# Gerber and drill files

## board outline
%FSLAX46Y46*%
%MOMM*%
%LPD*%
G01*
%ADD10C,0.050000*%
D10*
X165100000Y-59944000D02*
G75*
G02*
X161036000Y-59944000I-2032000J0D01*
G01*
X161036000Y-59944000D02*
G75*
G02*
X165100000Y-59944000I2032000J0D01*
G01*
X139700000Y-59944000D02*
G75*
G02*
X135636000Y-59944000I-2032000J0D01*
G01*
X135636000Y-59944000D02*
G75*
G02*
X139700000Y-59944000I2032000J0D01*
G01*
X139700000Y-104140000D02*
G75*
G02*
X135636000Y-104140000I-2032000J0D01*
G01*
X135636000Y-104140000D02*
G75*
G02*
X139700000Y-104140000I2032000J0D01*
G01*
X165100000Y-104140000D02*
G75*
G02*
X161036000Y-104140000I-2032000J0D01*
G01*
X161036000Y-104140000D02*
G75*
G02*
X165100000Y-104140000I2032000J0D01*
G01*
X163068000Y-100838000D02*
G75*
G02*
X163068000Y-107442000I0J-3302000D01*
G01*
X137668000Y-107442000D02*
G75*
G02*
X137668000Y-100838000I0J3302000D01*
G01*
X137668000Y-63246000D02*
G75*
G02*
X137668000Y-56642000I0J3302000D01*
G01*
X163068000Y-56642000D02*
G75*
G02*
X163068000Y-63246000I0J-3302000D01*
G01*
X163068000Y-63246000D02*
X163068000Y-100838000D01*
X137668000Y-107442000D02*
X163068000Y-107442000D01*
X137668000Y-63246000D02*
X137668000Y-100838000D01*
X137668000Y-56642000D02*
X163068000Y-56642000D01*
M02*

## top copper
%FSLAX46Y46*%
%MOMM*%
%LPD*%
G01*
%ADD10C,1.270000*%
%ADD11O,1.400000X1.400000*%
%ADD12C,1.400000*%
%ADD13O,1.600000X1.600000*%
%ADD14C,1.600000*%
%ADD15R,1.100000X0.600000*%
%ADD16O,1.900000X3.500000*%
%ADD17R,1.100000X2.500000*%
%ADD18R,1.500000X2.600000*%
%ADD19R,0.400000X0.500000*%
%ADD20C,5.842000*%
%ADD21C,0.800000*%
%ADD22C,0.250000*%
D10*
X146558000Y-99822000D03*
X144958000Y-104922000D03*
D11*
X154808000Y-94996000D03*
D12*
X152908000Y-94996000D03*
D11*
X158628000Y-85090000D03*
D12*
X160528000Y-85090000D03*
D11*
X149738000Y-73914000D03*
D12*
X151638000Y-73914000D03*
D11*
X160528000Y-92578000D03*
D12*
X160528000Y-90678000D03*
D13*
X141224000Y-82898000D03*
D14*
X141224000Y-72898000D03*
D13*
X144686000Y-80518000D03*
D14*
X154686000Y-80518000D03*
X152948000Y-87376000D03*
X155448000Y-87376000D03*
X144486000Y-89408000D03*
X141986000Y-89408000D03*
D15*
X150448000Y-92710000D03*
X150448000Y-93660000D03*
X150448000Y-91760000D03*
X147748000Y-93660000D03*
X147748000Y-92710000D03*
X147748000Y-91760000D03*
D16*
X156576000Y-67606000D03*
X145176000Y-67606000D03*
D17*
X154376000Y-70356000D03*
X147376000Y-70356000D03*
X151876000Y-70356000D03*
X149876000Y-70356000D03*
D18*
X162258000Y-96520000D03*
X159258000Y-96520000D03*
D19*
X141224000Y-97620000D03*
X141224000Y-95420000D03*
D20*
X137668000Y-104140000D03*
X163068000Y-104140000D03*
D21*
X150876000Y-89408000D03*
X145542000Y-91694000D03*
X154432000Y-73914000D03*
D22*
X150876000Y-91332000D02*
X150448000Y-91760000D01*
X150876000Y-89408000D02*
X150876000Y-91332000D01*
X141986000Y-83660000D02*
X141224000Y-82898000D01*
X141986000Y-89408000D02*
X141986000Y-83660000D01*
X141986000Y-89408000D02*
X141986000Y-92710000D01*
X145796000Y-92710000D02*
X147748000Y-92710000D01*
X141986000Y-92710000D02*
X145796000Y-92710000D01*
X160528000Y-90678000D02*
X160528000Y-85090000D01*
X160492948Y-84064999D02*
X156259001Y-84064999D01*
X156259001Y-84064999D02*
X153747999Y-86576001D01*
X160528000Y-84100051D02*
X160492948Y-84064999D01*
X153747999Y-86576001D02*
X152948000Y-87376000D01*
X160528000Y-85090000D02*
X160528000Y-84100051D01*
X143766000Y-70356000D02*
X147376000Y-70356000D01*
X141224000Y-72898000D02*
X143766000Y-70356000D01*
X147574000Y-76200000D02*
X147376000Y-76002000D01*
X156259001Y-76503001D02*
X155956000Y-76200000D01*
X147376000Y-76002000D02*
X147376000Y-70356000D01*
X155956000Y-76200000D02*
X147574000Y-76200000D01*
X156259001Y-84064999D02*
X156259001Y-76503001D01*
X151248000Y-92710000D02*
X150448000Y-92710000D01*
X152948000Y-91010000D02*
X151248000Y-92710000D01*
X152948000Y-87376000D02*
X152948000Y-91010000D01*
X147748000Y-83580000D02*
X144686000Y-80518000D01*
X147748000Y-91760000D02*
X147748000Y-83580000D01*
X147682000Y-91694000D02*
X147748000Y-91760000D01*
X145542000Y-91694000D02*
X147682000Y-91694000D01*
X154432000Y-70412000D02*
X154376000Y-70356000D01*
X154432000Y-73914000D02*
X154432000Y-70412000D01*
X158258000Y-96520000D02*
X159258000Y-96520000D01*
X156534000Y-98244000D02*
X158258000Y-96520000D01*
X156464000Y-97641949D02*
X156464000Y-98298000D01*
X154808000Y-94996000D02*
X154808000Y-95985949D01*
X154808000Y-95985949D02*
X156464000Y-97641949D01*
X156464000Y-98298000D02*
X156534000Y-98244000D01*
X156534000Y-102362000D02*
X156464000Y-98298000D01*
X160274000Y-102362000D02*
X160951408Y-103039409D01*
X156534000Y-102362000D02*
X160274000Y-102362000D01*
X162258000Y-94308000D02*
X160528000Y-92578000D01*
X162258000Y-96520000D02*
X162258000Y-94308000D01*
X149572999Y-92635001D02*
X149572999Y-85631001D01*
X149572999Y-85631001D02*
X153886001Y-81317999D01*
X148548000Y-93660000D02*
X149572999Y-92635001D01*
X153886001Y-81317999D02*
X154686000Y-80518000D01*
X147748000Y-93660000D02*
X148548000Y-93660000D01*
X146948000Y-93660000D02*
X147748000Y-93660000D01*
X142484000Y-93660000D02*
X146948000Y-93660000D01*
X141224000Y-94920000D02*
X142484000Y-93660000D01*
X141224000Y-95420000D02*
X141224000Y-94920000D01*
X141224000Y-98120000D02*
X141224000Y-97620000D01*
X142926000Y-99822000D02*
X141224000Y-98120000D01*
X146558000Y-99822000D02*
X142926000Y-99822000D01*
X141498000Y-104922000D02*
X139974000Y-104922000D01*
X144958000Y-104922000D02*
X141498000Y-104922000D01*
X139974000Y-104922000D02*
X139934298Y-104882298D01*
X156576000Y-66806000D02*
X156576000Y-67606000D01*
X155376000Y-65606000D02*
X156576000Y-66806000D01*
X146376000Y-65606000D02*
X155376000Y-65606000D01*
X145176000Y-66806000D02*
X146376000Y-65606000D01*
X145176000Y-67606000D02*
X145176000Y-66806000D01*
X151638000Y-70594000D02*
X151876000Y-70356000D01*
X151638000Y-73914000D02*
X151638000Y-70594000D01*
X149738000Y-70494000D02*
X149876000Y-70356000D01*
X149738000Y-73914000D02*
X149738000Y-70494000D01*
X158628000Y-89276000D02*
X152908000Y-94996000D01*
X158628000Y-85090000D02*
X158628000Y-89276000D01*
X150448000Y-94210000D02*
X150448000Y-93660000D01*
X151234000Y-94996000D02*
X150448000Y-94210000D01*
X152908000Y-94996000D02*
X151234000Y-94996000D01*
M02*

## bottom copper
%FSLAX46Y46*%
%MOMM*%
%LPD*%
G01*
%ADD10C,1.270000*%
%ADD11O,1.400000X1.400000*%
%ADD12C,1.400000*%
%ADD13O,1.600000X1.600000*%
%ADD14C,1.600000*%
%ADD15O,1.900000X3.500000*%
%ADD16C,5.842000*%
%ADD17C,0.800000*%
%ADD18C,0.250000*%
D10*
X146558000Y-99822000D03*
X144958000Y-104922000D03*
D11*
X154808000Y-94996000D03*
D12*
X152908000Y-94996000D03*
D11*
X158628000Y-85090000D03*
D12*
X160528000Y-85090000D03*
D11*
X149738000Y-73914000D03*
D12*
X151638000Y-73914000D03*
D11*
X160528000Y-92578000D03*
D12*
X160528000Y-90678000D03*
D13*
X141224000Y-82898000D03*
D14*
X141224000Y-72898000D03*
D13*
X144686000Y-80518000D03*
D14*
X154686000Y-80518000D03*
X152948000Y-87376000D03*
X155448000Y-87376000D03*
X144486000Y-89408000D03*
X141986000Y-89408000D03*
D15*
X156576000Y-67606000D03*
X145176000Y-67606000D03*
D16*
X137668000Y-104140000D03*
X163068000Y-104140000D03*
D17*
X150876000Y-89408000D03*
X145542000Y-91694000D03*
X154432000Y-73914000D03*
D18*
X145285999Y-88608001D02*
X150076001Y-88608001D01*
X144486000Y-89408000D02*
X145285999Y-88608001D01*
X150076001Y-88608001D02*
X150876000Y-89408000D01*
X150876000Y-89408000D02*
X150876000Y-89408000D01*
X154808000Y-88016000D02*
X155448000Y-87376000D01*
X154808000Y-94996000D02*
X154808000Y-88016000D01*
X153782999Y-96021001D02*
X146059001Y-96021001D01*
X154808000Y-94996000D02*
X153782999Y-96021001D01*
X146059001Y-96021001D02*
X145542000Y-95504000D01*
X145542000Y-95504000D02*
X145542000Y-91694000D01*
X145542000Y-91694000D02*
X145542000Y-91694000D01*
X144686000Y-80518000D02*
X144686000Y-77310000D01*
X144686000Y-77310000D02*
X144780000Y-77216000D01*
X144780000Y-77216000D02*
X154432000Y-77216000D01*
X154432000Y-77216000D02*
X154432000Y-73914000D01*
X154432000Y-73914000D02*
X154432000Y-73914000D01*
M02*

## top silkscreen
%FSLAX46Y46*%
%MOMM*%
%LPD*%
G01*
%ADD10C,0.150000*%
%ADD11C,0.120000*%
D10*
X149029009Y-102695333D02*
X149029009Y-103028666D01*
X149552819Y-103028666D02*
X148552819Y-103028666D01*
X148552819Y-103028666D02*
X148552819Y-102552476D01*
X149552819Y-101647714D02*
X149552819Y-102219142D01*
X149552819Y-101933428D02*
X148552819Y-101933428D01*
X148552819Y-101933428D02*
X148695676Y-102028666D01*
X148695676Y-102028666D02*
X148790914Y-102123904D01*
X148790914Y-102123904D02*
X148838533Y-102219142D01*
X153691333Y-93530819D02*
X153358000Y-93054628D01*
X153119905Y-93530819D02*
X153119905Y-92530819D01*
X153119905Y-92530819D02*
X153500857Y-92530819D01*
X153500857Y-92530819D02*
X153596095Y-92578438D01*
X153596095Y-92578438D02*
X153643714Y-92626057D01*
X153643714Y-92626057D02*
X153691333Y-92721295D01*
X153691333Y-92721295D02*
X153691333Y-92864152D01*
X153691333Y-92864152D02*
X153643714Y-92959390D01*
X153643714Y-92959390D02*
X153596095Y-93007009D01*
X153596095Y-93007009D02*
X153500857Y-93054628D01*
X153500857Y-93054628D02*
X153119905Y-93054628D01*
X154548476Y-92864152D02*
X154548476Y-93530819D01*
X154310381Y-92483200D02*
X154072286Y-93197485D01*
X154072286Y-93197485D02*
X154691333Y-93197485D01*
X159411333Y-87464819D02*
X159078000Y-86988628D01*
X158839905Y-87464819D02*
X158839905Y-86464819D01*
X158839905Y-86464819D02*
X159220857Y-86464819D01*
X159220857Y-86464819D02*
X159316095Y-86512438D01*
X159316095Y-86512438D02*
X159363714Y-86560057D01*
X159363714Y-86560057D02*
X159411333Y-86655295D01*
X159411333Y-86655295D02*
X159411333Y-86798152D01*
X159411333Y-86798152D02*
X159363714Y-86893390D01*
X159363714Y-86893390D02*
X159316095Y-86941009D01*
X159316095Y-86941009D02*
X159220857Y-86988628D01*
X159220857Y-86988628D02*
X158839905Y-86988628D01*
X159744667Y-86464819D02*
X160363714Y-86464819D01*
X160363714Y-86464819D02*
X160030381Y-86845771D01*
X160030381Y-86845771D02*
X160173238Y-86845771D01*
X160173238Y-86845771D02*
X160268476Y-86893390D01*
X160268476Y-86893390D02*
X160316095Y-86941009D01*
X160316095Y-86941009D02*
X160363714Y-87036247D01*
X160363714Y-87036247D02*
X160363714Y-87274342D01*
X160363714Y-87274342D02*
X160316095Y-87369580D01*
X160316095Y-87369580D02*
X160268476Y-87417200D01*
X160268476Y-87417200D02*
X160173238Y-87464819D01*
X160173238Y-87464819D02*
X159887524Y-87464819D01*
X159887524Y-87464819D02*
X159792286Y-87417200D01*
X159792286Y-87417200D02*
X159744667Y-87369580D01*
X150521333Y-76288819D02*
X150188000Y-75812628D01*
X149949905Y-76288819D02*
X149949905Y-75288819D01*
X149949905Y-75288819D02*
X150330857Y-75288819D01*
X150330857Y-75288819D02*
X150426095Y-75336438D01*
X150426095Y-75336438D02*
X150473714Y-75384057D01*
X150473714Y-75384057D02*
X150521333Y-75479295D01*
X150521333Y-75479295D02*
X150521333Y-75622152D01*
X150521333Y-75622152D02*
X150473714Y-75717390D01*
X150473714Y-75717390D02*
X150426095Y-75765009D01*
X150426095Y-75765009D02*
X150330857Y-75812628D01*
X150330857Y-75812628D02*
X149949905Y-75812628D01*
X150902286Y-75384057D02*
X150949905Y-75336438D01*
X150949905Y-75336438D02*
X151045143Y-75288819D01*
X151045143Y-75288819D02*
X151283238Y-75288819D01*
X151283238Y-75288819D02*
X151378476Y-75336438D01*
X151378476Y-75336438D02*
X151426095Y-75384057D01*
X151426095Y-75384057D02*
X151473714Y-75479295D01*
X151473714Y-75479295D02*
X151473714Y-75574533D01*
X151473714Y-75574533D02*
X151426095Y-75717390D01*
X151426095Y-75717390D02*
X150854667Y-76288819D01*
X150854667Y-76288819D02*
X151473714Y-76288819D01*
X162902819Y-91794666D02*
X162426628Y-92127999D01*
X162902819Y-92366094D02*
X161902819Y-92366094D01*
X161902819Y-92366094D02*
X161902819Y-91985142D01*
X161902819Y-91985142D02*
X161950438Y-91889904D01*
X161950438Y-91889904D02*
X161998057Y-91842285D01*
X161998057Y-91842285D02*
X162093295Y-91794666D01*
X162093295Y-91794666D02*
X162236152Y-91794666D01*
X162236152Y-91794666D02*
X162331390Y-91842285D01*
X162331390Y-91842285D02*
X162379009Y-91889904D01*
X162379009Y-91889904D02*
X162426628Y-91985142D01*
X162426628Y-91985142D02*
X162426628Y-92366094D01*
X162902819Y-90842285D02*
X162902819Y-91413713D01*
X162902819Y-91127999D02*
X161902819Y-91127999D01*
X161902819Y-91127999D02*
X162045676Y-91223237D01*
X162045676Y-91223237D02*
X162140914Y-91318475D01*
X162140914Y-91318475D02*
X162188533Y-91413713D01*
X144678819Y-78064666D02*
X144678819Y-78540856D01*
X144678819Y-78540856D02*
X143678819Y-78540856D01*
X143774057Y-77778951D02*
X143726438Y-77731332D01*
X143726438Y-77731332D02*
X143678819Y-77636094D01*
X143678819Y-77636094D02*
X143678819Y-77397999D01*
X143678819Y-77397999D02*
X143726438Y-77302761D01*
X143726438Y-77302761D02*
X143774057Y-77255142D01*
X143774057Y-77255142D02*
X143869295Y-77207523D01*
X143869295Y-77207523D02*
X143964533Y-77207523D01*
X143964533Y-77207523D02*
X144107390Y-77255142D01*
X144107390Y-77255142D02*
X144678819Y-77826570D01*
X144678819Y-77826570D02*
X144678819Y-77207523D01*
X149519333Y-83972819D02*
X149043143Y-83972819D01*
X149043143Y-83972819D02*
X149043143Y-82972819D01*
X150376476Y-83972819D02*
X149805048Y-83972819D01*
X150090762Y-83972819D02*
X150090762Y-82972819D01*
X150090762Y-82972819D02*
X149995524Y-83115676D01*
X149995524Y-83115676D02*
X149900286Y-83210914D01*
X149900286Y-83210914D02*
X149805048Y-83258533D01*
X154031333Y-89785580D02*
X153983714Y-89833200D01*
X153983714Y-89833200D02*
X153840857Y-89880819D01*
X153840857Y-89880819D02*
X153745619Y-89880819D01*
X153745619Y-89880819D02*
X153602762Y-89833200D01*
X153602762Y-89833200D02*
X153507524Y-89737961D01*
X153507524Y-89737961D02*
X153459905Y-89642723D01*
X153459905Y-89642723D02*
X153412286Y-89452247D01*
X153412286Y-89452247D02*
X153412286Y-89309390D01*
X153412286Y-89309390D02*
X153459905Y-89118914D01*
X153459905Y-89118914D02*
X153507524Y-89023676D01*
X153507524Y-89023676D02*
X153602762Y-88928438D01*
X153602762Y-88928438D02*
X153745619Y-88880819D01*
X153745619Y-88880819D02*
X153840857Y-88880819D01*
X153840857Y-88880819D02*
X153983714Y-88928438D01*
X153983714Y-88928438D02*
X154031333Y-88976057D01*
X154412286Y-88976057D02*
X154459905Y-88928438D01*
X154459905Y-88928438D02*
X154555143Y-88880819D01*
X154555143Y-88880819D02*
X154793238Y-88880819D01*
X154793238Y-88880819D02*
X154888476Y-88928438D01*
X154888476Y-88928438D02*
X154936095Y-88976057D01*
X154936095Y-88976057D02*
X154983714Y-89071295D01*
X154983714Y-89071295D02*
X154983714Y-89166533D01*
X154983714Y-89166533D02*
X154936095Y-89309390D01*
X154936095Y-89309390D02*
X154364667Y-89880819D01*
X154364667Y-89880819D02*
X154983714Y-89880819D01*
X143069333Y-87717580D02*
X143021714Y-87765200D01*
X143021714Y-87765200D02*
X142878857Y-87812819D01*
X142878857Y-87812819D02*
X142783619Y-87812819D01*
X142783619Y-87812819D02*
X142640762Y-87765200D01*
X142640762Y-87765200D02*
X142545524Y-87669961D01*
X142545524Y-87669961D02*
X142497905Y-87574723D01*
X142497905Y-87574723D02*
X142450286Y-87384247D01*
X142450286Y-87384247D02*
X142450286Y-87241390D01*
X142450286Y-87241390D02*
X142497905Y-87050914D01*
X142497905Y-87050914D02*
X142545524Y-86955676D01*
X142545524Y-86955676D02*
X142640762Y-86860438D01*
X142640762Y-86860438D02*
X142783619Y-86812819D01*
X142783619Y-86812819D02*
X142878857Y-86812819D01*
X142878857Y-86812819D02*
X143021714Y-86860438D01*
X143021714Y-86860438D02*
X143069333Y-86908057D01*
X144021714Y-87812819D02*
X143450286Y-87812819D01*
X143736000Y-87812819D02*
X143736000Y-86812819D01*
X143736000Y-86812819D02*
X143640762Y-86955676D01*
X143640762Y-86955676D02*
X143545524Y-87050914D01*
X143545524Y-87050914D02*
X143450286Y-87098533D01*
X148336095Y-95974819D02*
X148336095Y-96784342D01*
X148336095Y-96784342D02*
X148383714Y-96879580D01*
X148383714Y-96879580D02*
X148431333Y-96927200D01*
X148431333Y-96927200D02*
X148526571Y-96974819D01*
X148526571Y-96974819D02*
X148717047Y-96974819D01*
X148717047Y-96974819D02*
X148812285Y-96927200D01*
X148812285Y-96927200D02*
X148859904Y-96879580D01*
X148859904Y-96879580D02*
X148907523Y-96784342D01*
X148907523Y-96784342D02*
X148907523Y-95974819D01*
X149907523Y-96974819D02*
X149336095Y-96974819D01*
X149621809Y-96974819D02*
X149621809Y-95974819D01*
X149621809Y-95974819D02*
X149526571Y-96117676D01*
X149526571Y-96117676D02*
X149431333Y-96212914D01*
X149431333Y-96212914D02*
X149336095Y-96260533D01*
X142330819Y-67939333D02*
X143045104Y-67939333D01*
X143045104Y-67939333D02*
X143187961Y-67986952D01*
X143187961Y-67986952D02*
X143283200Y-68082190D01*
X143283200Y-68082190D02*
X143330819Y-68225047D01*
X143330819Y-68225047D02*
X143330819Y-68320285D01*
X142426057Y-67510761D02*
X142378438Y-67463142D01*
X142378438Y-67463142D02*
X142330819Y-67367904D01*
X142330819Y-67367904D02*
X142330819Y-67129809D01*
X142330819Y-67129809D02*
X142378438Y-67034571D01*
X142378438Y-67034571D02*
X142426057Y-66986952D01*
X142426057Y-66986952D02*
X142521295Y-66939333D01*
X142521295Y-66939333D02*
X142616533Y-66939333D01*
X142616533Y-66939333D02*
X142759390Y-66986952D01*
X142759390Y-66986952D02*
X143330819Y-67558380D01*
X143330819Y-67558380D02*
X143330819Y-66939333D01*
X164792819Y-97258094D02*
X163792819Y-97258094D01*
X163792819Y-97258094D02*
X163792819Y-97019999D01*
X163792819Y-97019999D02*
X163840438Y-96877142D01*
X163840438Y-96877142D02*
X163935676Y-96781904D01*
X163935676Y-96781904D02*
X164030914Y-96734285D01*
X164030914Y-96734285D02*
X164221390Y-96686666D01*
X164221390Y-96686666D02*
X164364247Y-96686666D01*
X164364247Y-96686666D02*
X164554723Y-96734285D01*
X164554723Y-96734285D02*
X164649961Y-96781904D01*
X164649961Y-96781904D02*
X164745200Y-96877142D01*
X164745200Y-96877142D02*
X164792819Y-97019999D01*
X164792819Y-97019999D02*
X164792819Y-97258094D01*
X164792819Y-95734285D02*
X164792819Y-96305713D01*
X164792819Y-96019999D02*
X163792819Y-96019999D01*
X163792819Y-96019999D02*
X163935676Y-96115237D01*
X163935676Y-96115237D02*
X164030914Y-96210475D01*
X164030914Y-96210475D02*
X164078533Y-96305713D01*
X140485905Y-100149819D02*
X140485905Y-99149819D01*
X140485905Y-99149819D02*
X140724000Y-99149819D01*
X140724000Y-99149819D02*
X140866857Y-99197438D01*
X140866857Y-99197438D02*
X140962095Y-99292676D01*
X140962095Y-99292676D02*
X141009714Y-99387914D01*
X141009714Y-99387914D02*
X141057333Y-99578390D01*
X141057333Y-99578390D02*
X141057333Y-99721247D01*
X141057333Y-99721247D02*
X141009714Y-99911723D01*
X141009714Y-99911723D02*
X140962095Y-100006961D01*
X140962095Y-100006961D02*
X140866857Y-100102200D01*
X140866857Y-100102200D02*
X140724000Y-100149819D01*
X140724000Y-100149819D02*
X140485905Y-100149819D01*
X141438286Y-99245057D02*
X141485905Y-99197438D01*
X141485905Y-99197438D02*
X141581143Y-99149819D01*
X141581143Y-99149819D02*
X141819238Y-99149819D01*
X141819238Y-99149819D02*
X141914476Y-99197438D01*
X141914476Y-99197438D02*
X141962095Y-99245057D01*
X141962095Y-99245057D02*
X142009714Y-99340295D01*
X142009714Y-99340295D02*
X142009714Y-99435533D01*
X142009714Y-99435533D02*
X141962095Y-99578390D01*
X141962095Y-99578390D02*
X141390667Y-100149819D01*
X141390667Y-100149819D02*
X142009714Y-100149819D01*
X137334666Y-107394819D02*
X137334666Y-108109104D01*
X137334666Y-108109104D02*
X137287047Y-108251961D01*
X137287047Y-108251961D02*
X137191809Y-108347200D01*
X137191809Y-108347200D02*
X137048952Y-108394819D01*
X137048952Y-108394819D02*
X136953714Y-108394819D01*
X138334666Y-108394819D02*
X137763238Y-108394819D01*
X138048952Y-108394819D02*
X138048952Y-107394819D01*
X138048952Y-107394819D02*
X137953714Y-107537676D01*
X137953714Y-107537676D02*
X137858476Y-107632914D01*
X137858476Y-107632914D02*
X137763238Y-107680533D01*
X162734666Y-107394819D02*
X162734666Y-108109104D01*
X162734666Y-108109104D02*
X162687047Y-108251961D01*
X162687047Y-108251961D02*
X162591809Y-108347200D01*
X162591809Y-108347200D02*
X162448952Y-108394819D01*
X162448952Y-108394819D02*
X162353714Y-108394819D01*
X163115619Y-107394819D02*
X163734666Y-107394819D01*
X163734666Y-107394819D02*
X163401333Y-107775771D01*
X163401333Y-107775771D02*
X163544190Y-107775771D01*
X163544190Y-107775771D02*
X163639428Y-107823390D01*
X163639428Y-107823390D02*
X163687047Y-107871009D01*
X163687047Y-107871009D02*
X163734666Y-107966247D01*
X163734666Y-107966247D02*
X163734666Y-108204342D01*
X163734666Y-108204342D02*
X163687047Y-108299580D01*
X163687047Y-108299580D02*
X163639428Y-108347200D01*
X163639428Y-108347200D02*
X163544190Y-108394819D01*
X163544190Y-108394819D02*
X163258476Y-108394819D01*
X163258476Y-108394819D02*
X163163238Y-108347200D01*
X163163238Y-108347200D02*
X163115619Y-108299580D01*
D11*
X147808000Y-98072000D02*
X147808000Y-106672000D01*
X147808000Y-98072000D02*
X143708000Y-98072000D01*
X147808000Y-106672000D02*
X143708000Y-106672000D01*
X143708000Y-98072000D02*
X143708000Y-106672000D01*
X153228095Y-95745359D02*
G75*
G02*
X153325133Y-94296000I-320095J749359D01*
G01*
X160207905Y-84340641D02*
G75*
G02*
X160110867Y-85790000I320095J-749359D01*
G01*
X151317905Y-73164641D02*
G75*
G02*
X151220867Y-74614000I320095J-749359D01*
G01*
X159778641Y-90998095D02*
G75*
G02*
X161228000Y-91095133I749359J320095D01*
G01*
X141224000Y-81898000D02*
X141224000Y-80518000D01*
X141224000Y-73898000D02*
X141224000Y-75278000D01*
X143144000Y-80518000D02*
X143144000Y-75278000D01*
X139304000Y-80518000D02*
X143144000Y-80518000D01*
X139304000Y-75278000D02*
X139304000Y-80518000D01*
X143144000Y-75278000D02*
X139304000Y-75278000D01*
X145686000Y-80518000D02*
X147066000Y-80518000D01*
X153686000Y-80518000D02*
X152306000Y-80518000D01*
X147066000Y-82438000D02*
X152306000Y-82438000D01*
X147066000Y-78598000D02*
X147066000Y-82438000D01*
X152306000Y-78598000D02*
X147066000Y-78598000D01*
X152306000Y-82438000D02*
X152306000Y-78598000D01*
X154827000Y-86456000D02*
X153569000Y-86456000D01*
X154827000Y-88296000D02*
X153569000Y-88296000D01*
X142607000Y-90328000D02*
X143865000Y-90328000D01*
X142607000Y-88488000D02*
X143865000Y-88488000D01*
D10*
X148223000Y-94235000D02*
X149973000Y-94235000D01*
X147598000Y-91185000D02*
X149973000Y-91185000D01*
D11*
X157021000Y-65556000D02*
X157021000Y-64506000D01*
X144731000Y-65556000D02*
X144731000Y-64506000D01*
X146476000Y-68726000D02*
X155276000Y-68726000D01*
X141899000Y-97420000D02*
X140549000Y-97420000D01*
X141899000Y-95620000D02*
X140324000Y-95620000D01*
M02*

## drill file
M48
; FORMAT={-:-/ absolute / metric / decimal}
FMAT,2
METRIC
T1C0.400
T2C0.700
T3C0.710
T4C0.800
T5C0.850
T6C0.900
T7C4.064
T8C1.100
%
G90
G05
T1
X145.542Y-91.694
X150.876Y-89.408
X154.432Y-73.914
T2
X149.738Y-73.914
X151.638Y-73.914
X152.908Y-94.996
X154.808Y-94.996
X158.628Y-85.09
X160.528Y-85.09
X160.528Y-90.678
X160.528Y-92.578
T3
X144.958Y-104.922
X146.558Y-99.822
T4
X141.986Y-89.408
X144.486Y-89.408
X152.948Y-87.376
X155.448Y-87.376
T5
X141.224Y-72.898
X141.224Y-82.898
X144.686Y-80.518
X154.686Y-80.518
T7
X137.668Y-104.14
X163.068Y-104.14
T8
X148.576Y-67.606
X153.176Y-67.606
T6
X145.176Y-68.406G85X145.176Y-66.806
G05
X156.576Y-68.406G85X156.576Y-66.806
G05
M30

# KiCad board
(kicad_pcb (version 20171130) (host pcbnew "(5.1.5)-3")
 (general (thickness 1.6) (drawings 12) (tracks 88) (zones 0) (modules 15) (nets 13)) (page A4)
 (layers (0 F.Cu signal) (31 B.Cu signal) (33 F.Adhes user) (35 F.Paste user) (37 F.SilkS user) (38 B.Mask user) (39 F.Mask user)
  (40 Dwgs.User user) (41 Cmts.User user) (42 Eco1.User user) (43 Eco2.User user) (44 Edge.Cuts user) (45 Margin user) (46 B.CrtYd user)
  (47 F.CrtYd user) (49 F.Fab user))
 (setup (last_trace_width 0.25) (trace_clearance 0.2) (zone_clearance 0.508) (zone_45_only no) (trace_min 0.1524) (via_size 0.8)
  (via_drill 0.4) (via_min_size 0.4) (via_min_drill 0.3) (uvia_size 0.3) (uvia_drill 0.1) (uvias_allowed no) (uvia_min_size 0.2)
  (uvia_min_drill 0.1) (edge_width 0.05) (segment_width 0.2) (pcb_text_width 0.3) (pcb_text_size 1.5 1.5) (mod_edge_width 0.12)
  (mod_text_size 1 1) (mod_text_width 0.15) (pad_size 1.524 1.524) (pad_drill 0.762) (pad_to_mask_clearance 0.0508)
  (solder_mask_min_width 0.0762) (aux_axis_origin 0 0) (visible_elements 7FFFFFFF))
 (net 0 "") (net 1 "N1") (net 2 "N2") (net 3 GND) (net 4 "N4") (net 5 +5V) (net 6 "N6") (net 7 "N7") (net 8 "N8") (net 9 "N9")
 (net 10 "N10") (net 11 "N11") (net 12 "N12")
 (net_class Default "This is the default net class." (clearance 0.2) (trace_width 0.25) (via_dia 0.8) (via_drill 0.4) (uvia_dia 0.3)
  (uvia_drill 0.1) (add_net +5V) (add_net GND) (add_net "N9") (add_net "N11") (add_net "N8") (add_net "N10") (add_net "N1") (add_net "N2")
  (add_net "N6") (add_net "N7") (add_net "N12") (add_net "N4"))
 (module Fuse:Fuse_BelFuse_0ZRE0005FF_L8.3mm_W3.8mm (layer F.Cu) (at 146.558 99.822 270)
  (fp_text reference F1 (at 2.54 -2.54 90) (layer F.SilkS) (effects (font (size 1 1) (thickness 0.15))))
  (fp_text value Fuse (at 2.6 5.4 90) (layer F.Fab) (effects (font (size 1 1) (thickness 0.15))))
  (fp_line (start -1.75 -1.25) (end 6.85 -1.25) (layer F.SilkS) (width 0.12))
  (fp_line (start -1.75 -1.25) (end -1.75 2.85) (layer F.SilkS) (width 0.12))
  (fp_line (start 6.85 -1.25) (end 6.85 2.85) (layer F.SilkS) (width 0.12))
  (fp_line (start -1.75 2.85) (end 6.85 2.85) (layer F.SilkS) (width 0.12))
  (pad 1 thru_hole circle (at 0 0 270) (size 1.27 1.27) (drill 0.71) (layers *.Cu *.Mask) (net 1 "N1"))
  (pad 2 thru_hole circle (at 5.1 1.6 270) (size 1.27 1.27) (drill 0.71) (layers *.Cu *.Mask) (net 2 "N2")))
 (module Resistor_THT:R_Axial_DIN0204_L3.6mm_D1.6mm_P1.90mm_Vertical (layer F.Cu) (at 152.908 94.996)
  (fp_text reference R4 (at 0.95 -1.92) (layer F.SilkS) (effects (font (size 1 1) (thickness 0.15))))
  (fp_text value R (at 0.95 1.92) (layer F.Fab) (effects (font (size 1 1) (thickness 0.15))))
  (fp_arc (start 0 0) (end 0.417133 -0.7) (angle -233.92106) (layer F.SilkS) (width 0.12))
  (pad 2 thru_hole oval (at 1.9 0) (size 1.4 1.4) (drill 0.7) (layers *.Cu *.Mask) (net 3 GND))
  (pad 1 thru_hole circle (at 0 0) (size 1.4 1.4) (drill 0.7) (layers *.Cu *.Mask) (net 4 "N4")))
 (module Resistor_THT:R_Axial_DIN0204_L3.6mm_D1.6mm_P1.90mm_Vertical (layer F.Cu) (at 160.528 85.09 180)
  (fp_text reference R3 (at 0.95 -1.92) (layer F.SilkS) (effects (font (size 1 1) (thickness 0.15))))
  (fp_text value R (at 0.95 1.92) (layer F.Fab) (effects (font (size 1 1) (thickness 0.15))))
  (fp_arc (start 0 0) (end 0.417133 -0.7) (angle -233.92106) (layer F.SilkS) (width 0.12))
  (pad 2 thru_hole oval (at 1.9 0 180) (size 1.4 1.4) (drill 0.7) (layers *.Cu *.Mask) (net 4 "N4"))
  (pad 1 thru_hole circle (at 0 0 180) (size 1.4 1.4) (drill 0.7) (layers *.Cu *.Mask) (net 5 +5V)))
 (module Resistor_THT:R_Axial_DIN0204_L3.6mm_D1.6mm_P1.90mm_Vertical (layer F.Cu) (at 151.638 73.914 180)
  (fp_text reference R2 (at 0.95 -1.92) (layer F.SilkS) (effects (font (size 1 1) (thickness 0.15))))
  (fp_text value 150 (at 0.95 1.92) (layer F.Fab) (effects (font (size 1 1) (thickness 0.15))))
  (fp_arc (start 0 0) (end 0.417133 -0.7) (angle -233.92106) (layer F.SilkS) (width 0.12))
  (pad 2 thru_hole oval (at 1.9 0 180) (size 1.4 1.4) (drill 0.7) (layers *.Cu *.Mask) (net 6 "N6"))
  (pad 1 thru_hole circle (at 0 0 180) (size 1.4 1.4) (drill 0.7) (layers *.Cu *.Mask) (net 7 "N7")))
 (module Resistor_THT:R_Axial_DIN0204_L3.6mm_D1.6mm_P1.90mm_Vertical (layer F.Cu) (at 160.528 90.678 270)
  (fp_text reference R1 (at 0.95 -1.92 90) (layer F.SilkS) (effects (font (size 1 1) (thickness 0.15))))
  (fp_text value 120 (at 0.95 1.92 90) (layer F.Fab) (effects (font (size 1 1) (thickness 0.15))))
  (fp_arc (start 0 0) (end 0.417133 -0.7) (angle -233.92106) (layer F.SilkS) (width 0.12))
  (pad 2 thru_hole oval (at 1.9 0 270) (size 1.4 1.4) (drill 0.7) (layers *.Cu *.Mask) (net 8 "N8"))
  (pad 1 thru_hole circle (at 0 0 270) (size 1.4 1.4) (drill 0.7) (layers *.Cu *.Mask) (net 5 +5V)))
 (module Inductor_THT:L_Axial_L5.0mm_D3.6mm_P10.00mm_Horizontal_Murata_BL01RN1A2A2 (layer F.Cu) (at 141.224 72.898 270)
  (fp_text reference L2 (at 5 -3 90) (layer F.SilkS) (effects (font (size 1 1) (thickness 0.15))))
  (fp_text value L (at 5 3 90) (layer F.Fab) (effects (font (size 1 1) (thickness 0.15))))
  (fp_line (start 9 0) (end 7.62 0) (layer F.SilkS) (width 0.12))
  (fp_line (start 1 0) (end 2.38 0) (layer F.SilkS) (width 0.12))
  (fp_line (start 7.62 -1.92) (end 2.38 -1.92) (layer F.SilkS) (width 0.12))
  (fp_line (start 7.62 1.92) (end 7.62 -1.92) (layer F.SilkS) (width 0.12))
  (fp_line (start 2.38 1.92) (end 7.62 1.92) (layer F.SilkS) (width 0.12))
  (fp_line (start 2.38 -1.92) (end 2.38 1.92) (layer F.SilkS) (width 0.12))
  (pad 2 thru_hole oval (at 10 0 270) (size 1.6 1.6) (drill 0.85) (layers *.Cu *.Mask) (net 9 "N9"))
  (pad 1 thru_hole circle (at 0 0 270) (size 1.6 1.6) (drill 0.85) (layers *.Cu *.Mask) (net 5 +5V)))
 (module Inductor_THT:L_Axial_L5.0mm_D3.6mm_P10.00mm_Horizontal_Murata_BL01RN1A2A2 (layer F.Cu) (at 154.686 80.518 180)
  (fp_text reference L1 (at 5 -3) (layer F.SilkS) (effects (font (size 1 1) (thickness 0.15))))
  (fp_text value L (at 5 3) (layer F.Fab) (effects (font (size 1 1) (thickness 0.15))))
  (fp_line (start 9 0) (end 7.62 0) (layer F.SilkS) (width 0.12))
  (fp_line (start 1 0) (end 2.38 0) (layer F.SilkS) (width 0.12))
  (fp_line (start 7.62 -1.92) (end 2.38 -1.92) (layer F.SilkS) (width 0.12))
  (fp_line (start 7.62 1.92) (end 7.62 -1.92) (layer F.SilkS) (width 0.12))
  (fp_line (start 2.38 1.92) (end 7.62 1.92) (layer F.SilkS) (width 0.12))
  (fp_line (start 2.38 -1.92) (end 2.38 1.92) (layer F.SilkS) (width 0.12))
  (pad 2 thru_hole oval (at 10 0 180) (size 1.6 1.6) (drill 0.85) (layers *.Cu *.Mask) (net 3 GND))
  (pad 1 thru_hole circle (at 0 0 180) (size 1.6 1.6) (drill 0.85) (layers *.Cu *.Mask) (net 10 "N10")))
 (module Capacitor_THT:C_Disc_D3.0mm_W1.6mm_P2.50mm (layer F.Cu) (at 155.448 87.376 180)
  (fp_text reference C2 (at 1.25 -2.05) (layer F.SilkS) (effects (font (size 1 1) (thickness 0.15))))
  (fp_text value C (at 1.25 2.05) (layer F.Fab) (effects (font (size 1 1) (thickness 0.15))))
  (fp_line (start 0.621 0.92) (end 1.879 0.92) (layer F.SilkS) (width 0.12))
  (fp_line (start 0.621 -0.92) (end 1.879 -0.92) (layer F.SilkS) (width 0.12))
  (pad 2 thru_hole circle (at 2.5 0 180) (size 1.6 1.6) (drill 0.8) (layers *.Cu *.Mask) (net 5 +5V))
  (pad 1 thru_hole circle (at 0 0 180) (size 1.6 1.6) (drill 0.8) (layers *.Cu *.Mask) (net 3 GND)))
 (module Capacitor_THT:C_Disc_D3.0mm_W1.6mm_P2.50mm (layer F.Cu) (at 141.986 89.408)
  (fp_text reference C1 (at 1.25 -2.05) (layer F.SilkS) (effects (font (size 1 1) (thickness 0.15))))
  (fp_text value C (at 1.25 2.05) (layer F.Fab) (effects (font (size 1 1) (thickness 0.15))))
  (fp_line (start 0.621 0.92) (end 1.879 0.92) (layer F.SilkS) (width 0.12))
  (fp_line (start 0.621 -0.92) (end 1.879 -0.92) (layer F.SilkS) (width 0.12))
  (pad 2 thru_hole circle (at 2.5 0) (size 1.6 1.6) (drill 0.8) (layers *.Cu *.Mask) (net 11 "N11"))
  (pad 1 thru_hole circle (at 0 0) (size 1.6 1.6) (drill 0.8) (layers *.Cu *.Mask) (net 9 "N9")))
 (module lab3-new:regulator (layer F.Cu) (at 149.098 92.71)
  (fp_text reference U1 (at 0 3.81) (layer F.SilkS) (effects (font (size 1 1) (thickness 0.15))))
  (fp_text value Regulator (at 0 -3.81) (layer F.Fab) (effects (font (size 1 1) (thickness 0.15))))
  (fp_line (start -0.875 1.525) (end 0.875 1.525) (layer F.SilkS) (width 0.15))
  (fp_line (start -1.5 -1.525) (end 0.875 -1.525) (layer F.SilkS) (width 0.15))
  (pad 5 smd rect (at 1.35 0) (size 1.1 0.6) (layers F.Cu F.Paste F.Mask) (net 5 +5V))
  (pad 4 smd rect (at 1.35 0.95) (size 1.1 0.6) (layers F.Cu F.Paste F.Mask) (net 4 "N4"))
  (pad 6 smd rect (at 1.35 -0.95) (size 1.1 0.6) (layers F.Cu F.Paste F.Mask) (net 11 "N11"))
  (pad 3 smd rect (at -1.35 0.95) (size 1.1 0.6) (layers F.Cu F.Paste F.Mask) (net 10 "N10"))
  (pad 2 smd rect (at -1.35 0) (size 1.1 0.6) (layers F.Cu F.Paste F.Mask) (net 9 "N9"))
  (pad 1 smd rect (at -1.35 -0.95) (size 1.1 0.6) (layers F.Cu F.Paste F.Mask) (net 3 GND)))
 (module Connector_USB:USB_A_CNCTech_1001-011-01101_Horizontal (layer F.Cu) (at 150.876 60.706 90)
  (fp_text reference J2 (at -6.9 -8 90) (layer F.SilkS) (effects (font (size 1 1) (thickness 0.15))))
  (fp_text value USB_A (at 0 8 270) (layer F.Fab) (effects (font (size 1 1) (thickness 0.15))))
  (fp_line (start -4.85 6.145) (end -3.8 6.145) (layer F.SilkS) (width 0.12))
  (fp_line (start -4.85 -6.145) (end -3.8 -6.145) (layer F.SilkS) (width 0.12))
  (fp_line (start -8.02 -4.4) (end -8.02 4.4) (layer F.SilkS) (width 0.12))
  (pad "" np_thru_hole circle (at -6.9 2.3 90) (size 1.1 1.1) (drill 1.1) (layers *.Cu *.Mask))
  (pad "" np_thru_hole circle (at -6.9 -2.3 90) (size 1.1 1.1) (drill 1.1) (layers *.Cu *.Mask))
  (pad 5 thru_hole oval (at -6.9 5.7 90) (size 3.5 1.9) (drill oval 2.5 0.9) (layers *.Cu *.Mask) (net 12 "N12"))
  (pad 5 thru_hole oval (at -6.9 -5.7 90) (size 3.5 1.9) (drill oval 2.5 0.9) (layers *.Cu *.Mask) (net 12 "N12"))
  (pad 4 smd rect (at -9.65 3.5 90) (size 2.5 1.1) (layers F.Cu F.Paste F.Mask) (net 3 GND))
  (pad 1 smd rect (at -9.65 -3.5 90) (size 2.5 1.1) (layers F.Cu F.Paste F.Mask) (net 5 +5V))
  (pad 3 smd rect (at -9.65 1 90) (size 2.5 1.1) (layers F.Cu F.Paste F.Mask) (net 7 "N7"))
  (pad 2 smd rect (at -9.65 -1 90) (size 2.5 1.1) (layers F.Cu F.Paste F.Mask) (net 6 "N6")))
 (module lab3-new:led (layer F.Cu) (at 159.258 96.52 90)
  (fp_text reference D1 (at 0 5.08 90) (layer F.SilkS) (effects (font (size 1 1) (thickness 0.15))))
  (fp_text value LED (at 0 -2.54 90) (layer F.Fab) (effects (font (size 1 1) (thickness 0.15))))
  (pad 2 smd rect (at 0 3 90) (size 2.6 1.5) (layers F.Cu F.Paste F.Mask) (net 8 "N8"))
  (pad 1 smd rect (at 0 0 90) (size 2.6 1.5) (layers F.Cu F.Paste F.Mask) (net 3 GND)))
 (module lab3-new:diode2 (layer F.Cu) (at 141.224 96.52)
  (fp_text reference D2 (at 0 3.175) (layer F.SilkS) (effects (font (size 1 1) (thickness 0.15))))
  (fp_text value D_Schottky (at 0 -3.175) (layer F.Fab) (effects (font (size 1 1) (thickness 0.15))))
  (fp_line (start 0.675 0.9) (end -0.675 0.9) (layer F.SilkS) (width 0.12))
  (fp_line (start 0.675 -0.9) (end -0.9 -0.9) (layer F.SilkS) (width 0.12))
  (pad 2 smd rect (at 0 1.1) (size 0.4 0.5) (layers F.Cu F.Paste F.Mask) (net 1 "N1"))
  (pad 1 smd rect (at 0 -1.1) (size 0.4 0.5) (layers F.Cu F.Paste F.Mask) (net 10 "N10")))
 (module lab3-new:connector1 (layer F.Cu) (at 137.668 104.14)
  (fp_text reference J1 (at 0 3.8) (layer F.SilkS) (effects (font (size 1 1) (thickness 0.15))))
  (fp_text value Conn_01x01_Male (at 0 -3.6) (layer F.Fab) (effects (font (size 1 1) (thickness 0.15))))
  (pad 1 thru_hole circle (at 0 0) (size 5.842 5.842) (drill 4.064) (layers *.Cu *.Mask) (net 2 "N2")))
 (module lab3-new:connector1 (layer F.Cu) (at 163.068 104.14)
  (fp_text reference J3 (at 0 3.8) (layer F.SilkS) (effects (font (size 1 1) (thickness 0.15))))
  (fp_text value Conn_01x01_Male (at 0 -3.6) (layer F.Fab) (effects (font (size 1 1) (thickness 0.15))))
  (pad 1 thru_hole circle (at 0 0) (size 5.842 5.842) (drill 4.064) (layers *.Cu *.Mask) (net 3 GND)))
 (gr_circle (center 163.068 59.944) (end 163.068 61.976) (layer Edge.Cuts) (width 0.05))
 (gr_circle (center 137.668 59.944) (end 137.668 61.976) (layer Edge.Cuts) (width 0.05))
 (gr_circle (center 137.668 104.14) (end 137.668 106.172) (layer Edge.Cuts) (width 0.05))
 (gr_circle (center 163.068 104.14) (end 163.068 106.172) (layer Edge.Cuts) (width 0.05))
 (gr_arc (start 163.068 104.14) (end 163.068 107.442) (angle -180) (layer Edge.Cuts) (width 0.05))
 (gr_arc (start 137.668 104.14) (end 137.668 100.838) (angle -180) (layer Edge.Cuts) (width 0.05))
 (gr_arc (start 137.668 59.944) (end 137.668 56.642) (angle -180) (layer Edge.Cuts) (width 0.05))
 (gr_arc (start 163.068 59.944) (end 163.068 63.246) (angle -180) (layer Edge.Cuts) (width 0.05))
 (gr_line (start 163.068 63.246) (end 163.068 100.838) (layer Edge.Cuts) (width 0.05))
 (gr_line (start 137.668 107.442) (end 163.068 107.442) (layer Edge.Cuts) (width 0.05))
 (gr_line (start 137.668 63.246) (end 137.668 100.838) (layer Edge.Cuts) (width 0.05))
 (gr_line (start 137.668 56.642) (end 163.068 56.642) (layer Edge.Cuts) (width 0.05))
 (segment (start 145.285999 88.608001) (end 150.076001 88.608001) (width 0.25) (layer B.Cu) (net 11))
 (segment (start 144.486 89.408) (end 145.285999 88.608001) (width 0.25) (layer B.Cu) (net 11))
 (segment (start 150.076001 88.608001) (end 150.876 89.408) (width 0.25) (layer B.Cu) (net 11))
 (segment (start 150.876 89.408) (end 150.876 89.408) (width 0.25) (layer B.Cu) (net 11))
 (via (at 150.876 89.408) (size 0.8) (drill 0.4) (layers F.Cu B.Cu) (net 11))
 (segment (start 150.876 91.332) (end 150.448 91.76) (width 0.25) (layer F.Cu) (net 11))
 (segment (start 150.876 89.408) (end 150.876 91.332) (width 0.25) (layer F.Cu) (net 11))
 (segment (start 141.986 83.66) (end 141.224 82.898) (width 0.25) (layer F.Cu) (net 9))
 (segment (start 141.986 89.408) (end 141.986 83.66) (width 0.25) (layer F.Cu) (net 9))
 (segment (start 141.986 89.408) (end 141.986 92.71) (width 0.25) (layer F.Cu) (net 9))
 (segment (start 145.796 92.71) (end 147.748 92.71) (width 0.25) (layer F.Cu) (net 9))
 (segment (start 141.986 92.71) (end 145.796 92.71) (width 0.25) (layer F.Cu) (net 9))
 (segment (start 160.528 90.678) (end 160.528 85.09) (width 0.25) (layer F.Cu) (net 5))
 (segment (start 160.492948 84.064999) (end 156.259001 84.064999) (width 0.25) (layer F.Cu) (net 5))
 (segment (start 156.259001 84.064999) (end 153.747999 86.576001) (width 0.25) (layer F.Cu) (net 5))
 (segment (start 160.528 84.100051) (end 160.492948 84.064999) (width 0.25) (layer F.Cu) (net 5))
 (segment (start 153.747999 86.576001) (end 152.948 87.376) (width 0.25) (layer F.Cu) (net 5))
 (segment (start 160.528 85.09) (end 160.528 84.100051) (width 0.25) (layer F.Cu) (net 5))
 (segment (start 143.766 70.356) (end 147.376 70.356) (width 0.25) (layer F.Cu) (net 5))
 (segment (start 141.224 72.898) (end 143.766 70.356) (width 0.25) (layer F.Cu) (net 5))
 (segment (start 147.574 76.2) (end 147.376 76.002) (width 0.25) (layer F.Cu) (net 5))
 (segment (start 156.259001 76.503001) (end 155.956 76.2) (width 0.25) (layer F.Cu) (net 5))
 (segment (start 147.376 76.002) (end 147.376 70.356) (width 0.25) (layer F.Cu) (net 5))
 (segment (start 155.956 76.2) (end 147.574 76.2) (width 0.25) (layer F.Cu) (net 5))
 (segment (start 156.259001 84.064999) (end 156.259001 76.503001) (width 0.25) (layer F.Cu) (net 5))
 (segment (start 151.248 92.71) (end 150.448 92.71) (width 0.25) (layer F.Cu) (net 5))
 (segment (start 152.948 91.01) (end 151.248 92.71) (width 0.25) (layer F.Cu) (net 5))
 (segment (start 152.948 87.376) (end 152.948 91.01) (width 0.25) (layer F.Cu) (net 5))
 (segment (start 154.808 88.016) (end 155.448 87.376) (width 0.25) (layer B.Cu) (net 3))
 (segment (start 154.808 94.996) (end 154.808 88.016) (width 0.25) (layer B.Cu) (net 3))
 (segment (start 147.748 83.58) (end 144.686 80.518) (width 0.25) (layer F.Cu) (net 3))
 (segment (start 147.748 91.76) (end 147.748 83.58) (width 0.25) (layer F.Cu) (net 3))
 (segment (start 153.782999 96.021001) (end 146.059001 96.021001) (width 0.25) (layer B.Cu) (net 3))
 (segment (start 154.808 94.996) (end 153.782999 96.021001) (width 0.25) (layer B.Cu) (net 3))
 (segment (start 146.059001 96.021001) (end 145.542 95.504) (width 0.25) (layer B.Cu) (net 3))
 (segment (start 145.542 95.504) (end 145.542 91.694) (width 0.25) (layer B.Cu) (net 3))
 (segment (start 145.542 91.694) (end 145.542 91.694) (width 0.25) (layer B.Cu) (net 3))
 (via (at 145.542 91.694) (size 0.8) (drill 0.4) (layers F.Cu B.Cu) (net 3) (status 1000000))
 (segment (start 147.682 91.694) (end 147.748 91.76) (width 0.25) (layer F.Cu) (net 3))
 (segment (start 145.542 91.694) (end 147.682 91.694) (width 0.25) (layer F.Cu) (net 3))
 (segment (start 144.686 80.518) (end 144.686 77.31) (width 0.25) (layer B.Cu) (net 3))
 (segment (start 144.686 77.31) (end 144.78 77.216) (width 0.25) (layer B.Cu) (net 3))
 (segment (start 144.78 77.216) (end 154.432 77.216) (width 0.25) (layer B.Cu) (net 3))
 (segment (start 154.432 77.216) (end 154.432 73.914) (width 0.25) (layer B.Cu) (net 3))
 (segment (start 154.432 73.914) (end 154.432 73.914) (width 0.25) (layer B.Cu) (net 3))
 (via (at 154.432 73.914) (size 0.8) (drill 0.4) (layers F.Cu B.Cu) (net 3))
 (segment (start 154.432 70.412) (end 154.376 70.356) (width 0.25) (layer F.Cu) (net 3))
 (segment (start 154.432 73.914) (end 154.432 70.412) (width 0.25) (layer F.Cu) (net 3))
 (segment (start 158.258 96.52) (end 159.258 96.52) (width 0.25) (layer F.Cu) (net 3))
 (segment (start 156.534 98.244) (end 158.258 96.52) (width 0.25) (layer F.Cu) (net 3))
 (segment (start 156.464 97.641949) (end 156.464 98.298) (width 0.25) (layer F.Cu) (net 3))
 (segment (start 154.808 94.996) (end 154.808 95.985949) (width 0.25) (layer F.Cu) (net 3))
 (segment (start 154.808 95.985949) (end 156.464 97.641949) (width 0.25) (layer F.Cu) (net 3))
 (segment (start 156.464 98.298) (end 156.534 98.244) (width 0.25) (layer F.Cu) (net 3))
 (segment (start 156.534 102.362) (end 156.464 98.298) (width 0.25) (layer F.Cu) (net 3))
 (segment (start 160.274 102.362) (end 160.951408 103.039409) (width 0.25) (layer F.Cu) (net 3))
 (segment (start 156.534 102.362) (end 160.274 102.362) (width 0.25) (layer F.Cu) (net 3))
 (segment (start 162.258 94.308) (end 160.528 92.578) (width 0.25) (layer F.Cu) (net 8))
 (segment (start 162.258 96.52) (end 162.258 94.308) (width 0.25) (layer F.Cu) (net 8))
 (segment (start 149.572999 92.635001) (end 149.572999 85.631001) (width 0.25) (layer F.Cu) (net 10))
 (segment (start 149.572999 85.631001) (end 153.886001 81.317999) (width 0.25) (layer F.Cu) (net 10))
 (segment (start 148.548 93.66) (end 149.572999 92.635001) (width 0.25) (layer F.Cu) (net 10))
 (segment (start 153.886001 81.317999) (end 154.686 80.518) (width 0.25) (layer F.Cu) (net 10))
 (segment (start 147.748 93.66) (end 148.548 93.66) (width 0.25) (layer F.Cu) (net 10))
 (segment (start 146.948 93.66) (end 147.748 93.66) (width 0.25) (layer F.Cu) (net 10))
 (segment (start 142.484 93.66) (end 146.948 93.66) (width 0.25) (layer F.Cu) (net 10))
 (segment (start 141.224 94.92) (end 142.484 93.66) (width 0.25) (layer F.Cu) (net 10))
 (segment (start 141.224 95.42) (end 141.224 94.92) (width 0.25) (layer F.Cu) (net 10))
 (segment (start 141.224 98.12) (end 141.224 97.62) (width 0.25) (layer F.Cu) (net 1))
 (segment (start 142.926 99.822) (end 141.224 98.12) (width 0.25) (layer F.Cu) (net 1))
 (segment (start 146.558 99.822) (end 142.926 99.822) (width 0.25) (layer F.Cu) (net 1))
 (segment (start 141.498 104.922) (end 139.974 104.922) (width 0.25) (layer F.Cu) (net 2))
 (segment (start 144.958 104.922) (end 141.498 104.922) (width 0.25) (layer F.Cu) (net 2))
 (segment (start 139.974 104.922) (end 139.934298 104.882298) (width 0.25) (layer F.Cu) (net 2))
 (segment (start 156.576 66.806) (end 156.576 67.606) (width 0.25) (layer F.Cu) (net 12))
 (segment (start 155.376 65.606) (end 156.576 66.806) (width 0.25) (layer F.Cu) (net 12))
 (segment (start 146.376 65.606) (end 155.376 65.606) (width 0.25) (layer F.Cu) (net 12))
 (segment (start 145.176 66.806) (end 146.376 65.606) (width 0.25) (layer F.Cu) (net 12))
 (segment (start 145.176 67.606) (end 145.176 66.806) (width 0.25) (layer F.Cu) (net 12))
 (segment (start 151.638 70.594) (end 151.876 70.356) (width 0.25) (layer F.Cu) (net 7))
 (segment (start 151.638 73.914) (end 151.638 70.594) (width 0.25) (layer F.Cu) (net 7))
 (segment (start 149.738 70.494) (end 149.876 70.356) (width 0.25) (layer F.Cu) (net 6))
 (segment (start 149.738 73.914) (end 149.738 70.494) (width 0.25) (layer F.Cu) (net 6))
 (segment (start 158.628 89.276) (end 152.908 94.996) (width 0.25) (layer F.Cu) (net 4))
 (segment (start 158.628 85.09) (end 158.628 89.276) (width 0.25) (layer F.Cu) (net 4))
 (segment (start 150.448 94.21) (end 150.448 93.66) (width 0.25) (layer F.Cu) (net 4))
 (segment (start 151.234 94.996) (end 150.448 94.21) (width 0.25) (layer F.Cu) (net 4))
 (segment (start 152.908 94.996) (end 151.234 94.996) (width 0.25) (layer F.Cu) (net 4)))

